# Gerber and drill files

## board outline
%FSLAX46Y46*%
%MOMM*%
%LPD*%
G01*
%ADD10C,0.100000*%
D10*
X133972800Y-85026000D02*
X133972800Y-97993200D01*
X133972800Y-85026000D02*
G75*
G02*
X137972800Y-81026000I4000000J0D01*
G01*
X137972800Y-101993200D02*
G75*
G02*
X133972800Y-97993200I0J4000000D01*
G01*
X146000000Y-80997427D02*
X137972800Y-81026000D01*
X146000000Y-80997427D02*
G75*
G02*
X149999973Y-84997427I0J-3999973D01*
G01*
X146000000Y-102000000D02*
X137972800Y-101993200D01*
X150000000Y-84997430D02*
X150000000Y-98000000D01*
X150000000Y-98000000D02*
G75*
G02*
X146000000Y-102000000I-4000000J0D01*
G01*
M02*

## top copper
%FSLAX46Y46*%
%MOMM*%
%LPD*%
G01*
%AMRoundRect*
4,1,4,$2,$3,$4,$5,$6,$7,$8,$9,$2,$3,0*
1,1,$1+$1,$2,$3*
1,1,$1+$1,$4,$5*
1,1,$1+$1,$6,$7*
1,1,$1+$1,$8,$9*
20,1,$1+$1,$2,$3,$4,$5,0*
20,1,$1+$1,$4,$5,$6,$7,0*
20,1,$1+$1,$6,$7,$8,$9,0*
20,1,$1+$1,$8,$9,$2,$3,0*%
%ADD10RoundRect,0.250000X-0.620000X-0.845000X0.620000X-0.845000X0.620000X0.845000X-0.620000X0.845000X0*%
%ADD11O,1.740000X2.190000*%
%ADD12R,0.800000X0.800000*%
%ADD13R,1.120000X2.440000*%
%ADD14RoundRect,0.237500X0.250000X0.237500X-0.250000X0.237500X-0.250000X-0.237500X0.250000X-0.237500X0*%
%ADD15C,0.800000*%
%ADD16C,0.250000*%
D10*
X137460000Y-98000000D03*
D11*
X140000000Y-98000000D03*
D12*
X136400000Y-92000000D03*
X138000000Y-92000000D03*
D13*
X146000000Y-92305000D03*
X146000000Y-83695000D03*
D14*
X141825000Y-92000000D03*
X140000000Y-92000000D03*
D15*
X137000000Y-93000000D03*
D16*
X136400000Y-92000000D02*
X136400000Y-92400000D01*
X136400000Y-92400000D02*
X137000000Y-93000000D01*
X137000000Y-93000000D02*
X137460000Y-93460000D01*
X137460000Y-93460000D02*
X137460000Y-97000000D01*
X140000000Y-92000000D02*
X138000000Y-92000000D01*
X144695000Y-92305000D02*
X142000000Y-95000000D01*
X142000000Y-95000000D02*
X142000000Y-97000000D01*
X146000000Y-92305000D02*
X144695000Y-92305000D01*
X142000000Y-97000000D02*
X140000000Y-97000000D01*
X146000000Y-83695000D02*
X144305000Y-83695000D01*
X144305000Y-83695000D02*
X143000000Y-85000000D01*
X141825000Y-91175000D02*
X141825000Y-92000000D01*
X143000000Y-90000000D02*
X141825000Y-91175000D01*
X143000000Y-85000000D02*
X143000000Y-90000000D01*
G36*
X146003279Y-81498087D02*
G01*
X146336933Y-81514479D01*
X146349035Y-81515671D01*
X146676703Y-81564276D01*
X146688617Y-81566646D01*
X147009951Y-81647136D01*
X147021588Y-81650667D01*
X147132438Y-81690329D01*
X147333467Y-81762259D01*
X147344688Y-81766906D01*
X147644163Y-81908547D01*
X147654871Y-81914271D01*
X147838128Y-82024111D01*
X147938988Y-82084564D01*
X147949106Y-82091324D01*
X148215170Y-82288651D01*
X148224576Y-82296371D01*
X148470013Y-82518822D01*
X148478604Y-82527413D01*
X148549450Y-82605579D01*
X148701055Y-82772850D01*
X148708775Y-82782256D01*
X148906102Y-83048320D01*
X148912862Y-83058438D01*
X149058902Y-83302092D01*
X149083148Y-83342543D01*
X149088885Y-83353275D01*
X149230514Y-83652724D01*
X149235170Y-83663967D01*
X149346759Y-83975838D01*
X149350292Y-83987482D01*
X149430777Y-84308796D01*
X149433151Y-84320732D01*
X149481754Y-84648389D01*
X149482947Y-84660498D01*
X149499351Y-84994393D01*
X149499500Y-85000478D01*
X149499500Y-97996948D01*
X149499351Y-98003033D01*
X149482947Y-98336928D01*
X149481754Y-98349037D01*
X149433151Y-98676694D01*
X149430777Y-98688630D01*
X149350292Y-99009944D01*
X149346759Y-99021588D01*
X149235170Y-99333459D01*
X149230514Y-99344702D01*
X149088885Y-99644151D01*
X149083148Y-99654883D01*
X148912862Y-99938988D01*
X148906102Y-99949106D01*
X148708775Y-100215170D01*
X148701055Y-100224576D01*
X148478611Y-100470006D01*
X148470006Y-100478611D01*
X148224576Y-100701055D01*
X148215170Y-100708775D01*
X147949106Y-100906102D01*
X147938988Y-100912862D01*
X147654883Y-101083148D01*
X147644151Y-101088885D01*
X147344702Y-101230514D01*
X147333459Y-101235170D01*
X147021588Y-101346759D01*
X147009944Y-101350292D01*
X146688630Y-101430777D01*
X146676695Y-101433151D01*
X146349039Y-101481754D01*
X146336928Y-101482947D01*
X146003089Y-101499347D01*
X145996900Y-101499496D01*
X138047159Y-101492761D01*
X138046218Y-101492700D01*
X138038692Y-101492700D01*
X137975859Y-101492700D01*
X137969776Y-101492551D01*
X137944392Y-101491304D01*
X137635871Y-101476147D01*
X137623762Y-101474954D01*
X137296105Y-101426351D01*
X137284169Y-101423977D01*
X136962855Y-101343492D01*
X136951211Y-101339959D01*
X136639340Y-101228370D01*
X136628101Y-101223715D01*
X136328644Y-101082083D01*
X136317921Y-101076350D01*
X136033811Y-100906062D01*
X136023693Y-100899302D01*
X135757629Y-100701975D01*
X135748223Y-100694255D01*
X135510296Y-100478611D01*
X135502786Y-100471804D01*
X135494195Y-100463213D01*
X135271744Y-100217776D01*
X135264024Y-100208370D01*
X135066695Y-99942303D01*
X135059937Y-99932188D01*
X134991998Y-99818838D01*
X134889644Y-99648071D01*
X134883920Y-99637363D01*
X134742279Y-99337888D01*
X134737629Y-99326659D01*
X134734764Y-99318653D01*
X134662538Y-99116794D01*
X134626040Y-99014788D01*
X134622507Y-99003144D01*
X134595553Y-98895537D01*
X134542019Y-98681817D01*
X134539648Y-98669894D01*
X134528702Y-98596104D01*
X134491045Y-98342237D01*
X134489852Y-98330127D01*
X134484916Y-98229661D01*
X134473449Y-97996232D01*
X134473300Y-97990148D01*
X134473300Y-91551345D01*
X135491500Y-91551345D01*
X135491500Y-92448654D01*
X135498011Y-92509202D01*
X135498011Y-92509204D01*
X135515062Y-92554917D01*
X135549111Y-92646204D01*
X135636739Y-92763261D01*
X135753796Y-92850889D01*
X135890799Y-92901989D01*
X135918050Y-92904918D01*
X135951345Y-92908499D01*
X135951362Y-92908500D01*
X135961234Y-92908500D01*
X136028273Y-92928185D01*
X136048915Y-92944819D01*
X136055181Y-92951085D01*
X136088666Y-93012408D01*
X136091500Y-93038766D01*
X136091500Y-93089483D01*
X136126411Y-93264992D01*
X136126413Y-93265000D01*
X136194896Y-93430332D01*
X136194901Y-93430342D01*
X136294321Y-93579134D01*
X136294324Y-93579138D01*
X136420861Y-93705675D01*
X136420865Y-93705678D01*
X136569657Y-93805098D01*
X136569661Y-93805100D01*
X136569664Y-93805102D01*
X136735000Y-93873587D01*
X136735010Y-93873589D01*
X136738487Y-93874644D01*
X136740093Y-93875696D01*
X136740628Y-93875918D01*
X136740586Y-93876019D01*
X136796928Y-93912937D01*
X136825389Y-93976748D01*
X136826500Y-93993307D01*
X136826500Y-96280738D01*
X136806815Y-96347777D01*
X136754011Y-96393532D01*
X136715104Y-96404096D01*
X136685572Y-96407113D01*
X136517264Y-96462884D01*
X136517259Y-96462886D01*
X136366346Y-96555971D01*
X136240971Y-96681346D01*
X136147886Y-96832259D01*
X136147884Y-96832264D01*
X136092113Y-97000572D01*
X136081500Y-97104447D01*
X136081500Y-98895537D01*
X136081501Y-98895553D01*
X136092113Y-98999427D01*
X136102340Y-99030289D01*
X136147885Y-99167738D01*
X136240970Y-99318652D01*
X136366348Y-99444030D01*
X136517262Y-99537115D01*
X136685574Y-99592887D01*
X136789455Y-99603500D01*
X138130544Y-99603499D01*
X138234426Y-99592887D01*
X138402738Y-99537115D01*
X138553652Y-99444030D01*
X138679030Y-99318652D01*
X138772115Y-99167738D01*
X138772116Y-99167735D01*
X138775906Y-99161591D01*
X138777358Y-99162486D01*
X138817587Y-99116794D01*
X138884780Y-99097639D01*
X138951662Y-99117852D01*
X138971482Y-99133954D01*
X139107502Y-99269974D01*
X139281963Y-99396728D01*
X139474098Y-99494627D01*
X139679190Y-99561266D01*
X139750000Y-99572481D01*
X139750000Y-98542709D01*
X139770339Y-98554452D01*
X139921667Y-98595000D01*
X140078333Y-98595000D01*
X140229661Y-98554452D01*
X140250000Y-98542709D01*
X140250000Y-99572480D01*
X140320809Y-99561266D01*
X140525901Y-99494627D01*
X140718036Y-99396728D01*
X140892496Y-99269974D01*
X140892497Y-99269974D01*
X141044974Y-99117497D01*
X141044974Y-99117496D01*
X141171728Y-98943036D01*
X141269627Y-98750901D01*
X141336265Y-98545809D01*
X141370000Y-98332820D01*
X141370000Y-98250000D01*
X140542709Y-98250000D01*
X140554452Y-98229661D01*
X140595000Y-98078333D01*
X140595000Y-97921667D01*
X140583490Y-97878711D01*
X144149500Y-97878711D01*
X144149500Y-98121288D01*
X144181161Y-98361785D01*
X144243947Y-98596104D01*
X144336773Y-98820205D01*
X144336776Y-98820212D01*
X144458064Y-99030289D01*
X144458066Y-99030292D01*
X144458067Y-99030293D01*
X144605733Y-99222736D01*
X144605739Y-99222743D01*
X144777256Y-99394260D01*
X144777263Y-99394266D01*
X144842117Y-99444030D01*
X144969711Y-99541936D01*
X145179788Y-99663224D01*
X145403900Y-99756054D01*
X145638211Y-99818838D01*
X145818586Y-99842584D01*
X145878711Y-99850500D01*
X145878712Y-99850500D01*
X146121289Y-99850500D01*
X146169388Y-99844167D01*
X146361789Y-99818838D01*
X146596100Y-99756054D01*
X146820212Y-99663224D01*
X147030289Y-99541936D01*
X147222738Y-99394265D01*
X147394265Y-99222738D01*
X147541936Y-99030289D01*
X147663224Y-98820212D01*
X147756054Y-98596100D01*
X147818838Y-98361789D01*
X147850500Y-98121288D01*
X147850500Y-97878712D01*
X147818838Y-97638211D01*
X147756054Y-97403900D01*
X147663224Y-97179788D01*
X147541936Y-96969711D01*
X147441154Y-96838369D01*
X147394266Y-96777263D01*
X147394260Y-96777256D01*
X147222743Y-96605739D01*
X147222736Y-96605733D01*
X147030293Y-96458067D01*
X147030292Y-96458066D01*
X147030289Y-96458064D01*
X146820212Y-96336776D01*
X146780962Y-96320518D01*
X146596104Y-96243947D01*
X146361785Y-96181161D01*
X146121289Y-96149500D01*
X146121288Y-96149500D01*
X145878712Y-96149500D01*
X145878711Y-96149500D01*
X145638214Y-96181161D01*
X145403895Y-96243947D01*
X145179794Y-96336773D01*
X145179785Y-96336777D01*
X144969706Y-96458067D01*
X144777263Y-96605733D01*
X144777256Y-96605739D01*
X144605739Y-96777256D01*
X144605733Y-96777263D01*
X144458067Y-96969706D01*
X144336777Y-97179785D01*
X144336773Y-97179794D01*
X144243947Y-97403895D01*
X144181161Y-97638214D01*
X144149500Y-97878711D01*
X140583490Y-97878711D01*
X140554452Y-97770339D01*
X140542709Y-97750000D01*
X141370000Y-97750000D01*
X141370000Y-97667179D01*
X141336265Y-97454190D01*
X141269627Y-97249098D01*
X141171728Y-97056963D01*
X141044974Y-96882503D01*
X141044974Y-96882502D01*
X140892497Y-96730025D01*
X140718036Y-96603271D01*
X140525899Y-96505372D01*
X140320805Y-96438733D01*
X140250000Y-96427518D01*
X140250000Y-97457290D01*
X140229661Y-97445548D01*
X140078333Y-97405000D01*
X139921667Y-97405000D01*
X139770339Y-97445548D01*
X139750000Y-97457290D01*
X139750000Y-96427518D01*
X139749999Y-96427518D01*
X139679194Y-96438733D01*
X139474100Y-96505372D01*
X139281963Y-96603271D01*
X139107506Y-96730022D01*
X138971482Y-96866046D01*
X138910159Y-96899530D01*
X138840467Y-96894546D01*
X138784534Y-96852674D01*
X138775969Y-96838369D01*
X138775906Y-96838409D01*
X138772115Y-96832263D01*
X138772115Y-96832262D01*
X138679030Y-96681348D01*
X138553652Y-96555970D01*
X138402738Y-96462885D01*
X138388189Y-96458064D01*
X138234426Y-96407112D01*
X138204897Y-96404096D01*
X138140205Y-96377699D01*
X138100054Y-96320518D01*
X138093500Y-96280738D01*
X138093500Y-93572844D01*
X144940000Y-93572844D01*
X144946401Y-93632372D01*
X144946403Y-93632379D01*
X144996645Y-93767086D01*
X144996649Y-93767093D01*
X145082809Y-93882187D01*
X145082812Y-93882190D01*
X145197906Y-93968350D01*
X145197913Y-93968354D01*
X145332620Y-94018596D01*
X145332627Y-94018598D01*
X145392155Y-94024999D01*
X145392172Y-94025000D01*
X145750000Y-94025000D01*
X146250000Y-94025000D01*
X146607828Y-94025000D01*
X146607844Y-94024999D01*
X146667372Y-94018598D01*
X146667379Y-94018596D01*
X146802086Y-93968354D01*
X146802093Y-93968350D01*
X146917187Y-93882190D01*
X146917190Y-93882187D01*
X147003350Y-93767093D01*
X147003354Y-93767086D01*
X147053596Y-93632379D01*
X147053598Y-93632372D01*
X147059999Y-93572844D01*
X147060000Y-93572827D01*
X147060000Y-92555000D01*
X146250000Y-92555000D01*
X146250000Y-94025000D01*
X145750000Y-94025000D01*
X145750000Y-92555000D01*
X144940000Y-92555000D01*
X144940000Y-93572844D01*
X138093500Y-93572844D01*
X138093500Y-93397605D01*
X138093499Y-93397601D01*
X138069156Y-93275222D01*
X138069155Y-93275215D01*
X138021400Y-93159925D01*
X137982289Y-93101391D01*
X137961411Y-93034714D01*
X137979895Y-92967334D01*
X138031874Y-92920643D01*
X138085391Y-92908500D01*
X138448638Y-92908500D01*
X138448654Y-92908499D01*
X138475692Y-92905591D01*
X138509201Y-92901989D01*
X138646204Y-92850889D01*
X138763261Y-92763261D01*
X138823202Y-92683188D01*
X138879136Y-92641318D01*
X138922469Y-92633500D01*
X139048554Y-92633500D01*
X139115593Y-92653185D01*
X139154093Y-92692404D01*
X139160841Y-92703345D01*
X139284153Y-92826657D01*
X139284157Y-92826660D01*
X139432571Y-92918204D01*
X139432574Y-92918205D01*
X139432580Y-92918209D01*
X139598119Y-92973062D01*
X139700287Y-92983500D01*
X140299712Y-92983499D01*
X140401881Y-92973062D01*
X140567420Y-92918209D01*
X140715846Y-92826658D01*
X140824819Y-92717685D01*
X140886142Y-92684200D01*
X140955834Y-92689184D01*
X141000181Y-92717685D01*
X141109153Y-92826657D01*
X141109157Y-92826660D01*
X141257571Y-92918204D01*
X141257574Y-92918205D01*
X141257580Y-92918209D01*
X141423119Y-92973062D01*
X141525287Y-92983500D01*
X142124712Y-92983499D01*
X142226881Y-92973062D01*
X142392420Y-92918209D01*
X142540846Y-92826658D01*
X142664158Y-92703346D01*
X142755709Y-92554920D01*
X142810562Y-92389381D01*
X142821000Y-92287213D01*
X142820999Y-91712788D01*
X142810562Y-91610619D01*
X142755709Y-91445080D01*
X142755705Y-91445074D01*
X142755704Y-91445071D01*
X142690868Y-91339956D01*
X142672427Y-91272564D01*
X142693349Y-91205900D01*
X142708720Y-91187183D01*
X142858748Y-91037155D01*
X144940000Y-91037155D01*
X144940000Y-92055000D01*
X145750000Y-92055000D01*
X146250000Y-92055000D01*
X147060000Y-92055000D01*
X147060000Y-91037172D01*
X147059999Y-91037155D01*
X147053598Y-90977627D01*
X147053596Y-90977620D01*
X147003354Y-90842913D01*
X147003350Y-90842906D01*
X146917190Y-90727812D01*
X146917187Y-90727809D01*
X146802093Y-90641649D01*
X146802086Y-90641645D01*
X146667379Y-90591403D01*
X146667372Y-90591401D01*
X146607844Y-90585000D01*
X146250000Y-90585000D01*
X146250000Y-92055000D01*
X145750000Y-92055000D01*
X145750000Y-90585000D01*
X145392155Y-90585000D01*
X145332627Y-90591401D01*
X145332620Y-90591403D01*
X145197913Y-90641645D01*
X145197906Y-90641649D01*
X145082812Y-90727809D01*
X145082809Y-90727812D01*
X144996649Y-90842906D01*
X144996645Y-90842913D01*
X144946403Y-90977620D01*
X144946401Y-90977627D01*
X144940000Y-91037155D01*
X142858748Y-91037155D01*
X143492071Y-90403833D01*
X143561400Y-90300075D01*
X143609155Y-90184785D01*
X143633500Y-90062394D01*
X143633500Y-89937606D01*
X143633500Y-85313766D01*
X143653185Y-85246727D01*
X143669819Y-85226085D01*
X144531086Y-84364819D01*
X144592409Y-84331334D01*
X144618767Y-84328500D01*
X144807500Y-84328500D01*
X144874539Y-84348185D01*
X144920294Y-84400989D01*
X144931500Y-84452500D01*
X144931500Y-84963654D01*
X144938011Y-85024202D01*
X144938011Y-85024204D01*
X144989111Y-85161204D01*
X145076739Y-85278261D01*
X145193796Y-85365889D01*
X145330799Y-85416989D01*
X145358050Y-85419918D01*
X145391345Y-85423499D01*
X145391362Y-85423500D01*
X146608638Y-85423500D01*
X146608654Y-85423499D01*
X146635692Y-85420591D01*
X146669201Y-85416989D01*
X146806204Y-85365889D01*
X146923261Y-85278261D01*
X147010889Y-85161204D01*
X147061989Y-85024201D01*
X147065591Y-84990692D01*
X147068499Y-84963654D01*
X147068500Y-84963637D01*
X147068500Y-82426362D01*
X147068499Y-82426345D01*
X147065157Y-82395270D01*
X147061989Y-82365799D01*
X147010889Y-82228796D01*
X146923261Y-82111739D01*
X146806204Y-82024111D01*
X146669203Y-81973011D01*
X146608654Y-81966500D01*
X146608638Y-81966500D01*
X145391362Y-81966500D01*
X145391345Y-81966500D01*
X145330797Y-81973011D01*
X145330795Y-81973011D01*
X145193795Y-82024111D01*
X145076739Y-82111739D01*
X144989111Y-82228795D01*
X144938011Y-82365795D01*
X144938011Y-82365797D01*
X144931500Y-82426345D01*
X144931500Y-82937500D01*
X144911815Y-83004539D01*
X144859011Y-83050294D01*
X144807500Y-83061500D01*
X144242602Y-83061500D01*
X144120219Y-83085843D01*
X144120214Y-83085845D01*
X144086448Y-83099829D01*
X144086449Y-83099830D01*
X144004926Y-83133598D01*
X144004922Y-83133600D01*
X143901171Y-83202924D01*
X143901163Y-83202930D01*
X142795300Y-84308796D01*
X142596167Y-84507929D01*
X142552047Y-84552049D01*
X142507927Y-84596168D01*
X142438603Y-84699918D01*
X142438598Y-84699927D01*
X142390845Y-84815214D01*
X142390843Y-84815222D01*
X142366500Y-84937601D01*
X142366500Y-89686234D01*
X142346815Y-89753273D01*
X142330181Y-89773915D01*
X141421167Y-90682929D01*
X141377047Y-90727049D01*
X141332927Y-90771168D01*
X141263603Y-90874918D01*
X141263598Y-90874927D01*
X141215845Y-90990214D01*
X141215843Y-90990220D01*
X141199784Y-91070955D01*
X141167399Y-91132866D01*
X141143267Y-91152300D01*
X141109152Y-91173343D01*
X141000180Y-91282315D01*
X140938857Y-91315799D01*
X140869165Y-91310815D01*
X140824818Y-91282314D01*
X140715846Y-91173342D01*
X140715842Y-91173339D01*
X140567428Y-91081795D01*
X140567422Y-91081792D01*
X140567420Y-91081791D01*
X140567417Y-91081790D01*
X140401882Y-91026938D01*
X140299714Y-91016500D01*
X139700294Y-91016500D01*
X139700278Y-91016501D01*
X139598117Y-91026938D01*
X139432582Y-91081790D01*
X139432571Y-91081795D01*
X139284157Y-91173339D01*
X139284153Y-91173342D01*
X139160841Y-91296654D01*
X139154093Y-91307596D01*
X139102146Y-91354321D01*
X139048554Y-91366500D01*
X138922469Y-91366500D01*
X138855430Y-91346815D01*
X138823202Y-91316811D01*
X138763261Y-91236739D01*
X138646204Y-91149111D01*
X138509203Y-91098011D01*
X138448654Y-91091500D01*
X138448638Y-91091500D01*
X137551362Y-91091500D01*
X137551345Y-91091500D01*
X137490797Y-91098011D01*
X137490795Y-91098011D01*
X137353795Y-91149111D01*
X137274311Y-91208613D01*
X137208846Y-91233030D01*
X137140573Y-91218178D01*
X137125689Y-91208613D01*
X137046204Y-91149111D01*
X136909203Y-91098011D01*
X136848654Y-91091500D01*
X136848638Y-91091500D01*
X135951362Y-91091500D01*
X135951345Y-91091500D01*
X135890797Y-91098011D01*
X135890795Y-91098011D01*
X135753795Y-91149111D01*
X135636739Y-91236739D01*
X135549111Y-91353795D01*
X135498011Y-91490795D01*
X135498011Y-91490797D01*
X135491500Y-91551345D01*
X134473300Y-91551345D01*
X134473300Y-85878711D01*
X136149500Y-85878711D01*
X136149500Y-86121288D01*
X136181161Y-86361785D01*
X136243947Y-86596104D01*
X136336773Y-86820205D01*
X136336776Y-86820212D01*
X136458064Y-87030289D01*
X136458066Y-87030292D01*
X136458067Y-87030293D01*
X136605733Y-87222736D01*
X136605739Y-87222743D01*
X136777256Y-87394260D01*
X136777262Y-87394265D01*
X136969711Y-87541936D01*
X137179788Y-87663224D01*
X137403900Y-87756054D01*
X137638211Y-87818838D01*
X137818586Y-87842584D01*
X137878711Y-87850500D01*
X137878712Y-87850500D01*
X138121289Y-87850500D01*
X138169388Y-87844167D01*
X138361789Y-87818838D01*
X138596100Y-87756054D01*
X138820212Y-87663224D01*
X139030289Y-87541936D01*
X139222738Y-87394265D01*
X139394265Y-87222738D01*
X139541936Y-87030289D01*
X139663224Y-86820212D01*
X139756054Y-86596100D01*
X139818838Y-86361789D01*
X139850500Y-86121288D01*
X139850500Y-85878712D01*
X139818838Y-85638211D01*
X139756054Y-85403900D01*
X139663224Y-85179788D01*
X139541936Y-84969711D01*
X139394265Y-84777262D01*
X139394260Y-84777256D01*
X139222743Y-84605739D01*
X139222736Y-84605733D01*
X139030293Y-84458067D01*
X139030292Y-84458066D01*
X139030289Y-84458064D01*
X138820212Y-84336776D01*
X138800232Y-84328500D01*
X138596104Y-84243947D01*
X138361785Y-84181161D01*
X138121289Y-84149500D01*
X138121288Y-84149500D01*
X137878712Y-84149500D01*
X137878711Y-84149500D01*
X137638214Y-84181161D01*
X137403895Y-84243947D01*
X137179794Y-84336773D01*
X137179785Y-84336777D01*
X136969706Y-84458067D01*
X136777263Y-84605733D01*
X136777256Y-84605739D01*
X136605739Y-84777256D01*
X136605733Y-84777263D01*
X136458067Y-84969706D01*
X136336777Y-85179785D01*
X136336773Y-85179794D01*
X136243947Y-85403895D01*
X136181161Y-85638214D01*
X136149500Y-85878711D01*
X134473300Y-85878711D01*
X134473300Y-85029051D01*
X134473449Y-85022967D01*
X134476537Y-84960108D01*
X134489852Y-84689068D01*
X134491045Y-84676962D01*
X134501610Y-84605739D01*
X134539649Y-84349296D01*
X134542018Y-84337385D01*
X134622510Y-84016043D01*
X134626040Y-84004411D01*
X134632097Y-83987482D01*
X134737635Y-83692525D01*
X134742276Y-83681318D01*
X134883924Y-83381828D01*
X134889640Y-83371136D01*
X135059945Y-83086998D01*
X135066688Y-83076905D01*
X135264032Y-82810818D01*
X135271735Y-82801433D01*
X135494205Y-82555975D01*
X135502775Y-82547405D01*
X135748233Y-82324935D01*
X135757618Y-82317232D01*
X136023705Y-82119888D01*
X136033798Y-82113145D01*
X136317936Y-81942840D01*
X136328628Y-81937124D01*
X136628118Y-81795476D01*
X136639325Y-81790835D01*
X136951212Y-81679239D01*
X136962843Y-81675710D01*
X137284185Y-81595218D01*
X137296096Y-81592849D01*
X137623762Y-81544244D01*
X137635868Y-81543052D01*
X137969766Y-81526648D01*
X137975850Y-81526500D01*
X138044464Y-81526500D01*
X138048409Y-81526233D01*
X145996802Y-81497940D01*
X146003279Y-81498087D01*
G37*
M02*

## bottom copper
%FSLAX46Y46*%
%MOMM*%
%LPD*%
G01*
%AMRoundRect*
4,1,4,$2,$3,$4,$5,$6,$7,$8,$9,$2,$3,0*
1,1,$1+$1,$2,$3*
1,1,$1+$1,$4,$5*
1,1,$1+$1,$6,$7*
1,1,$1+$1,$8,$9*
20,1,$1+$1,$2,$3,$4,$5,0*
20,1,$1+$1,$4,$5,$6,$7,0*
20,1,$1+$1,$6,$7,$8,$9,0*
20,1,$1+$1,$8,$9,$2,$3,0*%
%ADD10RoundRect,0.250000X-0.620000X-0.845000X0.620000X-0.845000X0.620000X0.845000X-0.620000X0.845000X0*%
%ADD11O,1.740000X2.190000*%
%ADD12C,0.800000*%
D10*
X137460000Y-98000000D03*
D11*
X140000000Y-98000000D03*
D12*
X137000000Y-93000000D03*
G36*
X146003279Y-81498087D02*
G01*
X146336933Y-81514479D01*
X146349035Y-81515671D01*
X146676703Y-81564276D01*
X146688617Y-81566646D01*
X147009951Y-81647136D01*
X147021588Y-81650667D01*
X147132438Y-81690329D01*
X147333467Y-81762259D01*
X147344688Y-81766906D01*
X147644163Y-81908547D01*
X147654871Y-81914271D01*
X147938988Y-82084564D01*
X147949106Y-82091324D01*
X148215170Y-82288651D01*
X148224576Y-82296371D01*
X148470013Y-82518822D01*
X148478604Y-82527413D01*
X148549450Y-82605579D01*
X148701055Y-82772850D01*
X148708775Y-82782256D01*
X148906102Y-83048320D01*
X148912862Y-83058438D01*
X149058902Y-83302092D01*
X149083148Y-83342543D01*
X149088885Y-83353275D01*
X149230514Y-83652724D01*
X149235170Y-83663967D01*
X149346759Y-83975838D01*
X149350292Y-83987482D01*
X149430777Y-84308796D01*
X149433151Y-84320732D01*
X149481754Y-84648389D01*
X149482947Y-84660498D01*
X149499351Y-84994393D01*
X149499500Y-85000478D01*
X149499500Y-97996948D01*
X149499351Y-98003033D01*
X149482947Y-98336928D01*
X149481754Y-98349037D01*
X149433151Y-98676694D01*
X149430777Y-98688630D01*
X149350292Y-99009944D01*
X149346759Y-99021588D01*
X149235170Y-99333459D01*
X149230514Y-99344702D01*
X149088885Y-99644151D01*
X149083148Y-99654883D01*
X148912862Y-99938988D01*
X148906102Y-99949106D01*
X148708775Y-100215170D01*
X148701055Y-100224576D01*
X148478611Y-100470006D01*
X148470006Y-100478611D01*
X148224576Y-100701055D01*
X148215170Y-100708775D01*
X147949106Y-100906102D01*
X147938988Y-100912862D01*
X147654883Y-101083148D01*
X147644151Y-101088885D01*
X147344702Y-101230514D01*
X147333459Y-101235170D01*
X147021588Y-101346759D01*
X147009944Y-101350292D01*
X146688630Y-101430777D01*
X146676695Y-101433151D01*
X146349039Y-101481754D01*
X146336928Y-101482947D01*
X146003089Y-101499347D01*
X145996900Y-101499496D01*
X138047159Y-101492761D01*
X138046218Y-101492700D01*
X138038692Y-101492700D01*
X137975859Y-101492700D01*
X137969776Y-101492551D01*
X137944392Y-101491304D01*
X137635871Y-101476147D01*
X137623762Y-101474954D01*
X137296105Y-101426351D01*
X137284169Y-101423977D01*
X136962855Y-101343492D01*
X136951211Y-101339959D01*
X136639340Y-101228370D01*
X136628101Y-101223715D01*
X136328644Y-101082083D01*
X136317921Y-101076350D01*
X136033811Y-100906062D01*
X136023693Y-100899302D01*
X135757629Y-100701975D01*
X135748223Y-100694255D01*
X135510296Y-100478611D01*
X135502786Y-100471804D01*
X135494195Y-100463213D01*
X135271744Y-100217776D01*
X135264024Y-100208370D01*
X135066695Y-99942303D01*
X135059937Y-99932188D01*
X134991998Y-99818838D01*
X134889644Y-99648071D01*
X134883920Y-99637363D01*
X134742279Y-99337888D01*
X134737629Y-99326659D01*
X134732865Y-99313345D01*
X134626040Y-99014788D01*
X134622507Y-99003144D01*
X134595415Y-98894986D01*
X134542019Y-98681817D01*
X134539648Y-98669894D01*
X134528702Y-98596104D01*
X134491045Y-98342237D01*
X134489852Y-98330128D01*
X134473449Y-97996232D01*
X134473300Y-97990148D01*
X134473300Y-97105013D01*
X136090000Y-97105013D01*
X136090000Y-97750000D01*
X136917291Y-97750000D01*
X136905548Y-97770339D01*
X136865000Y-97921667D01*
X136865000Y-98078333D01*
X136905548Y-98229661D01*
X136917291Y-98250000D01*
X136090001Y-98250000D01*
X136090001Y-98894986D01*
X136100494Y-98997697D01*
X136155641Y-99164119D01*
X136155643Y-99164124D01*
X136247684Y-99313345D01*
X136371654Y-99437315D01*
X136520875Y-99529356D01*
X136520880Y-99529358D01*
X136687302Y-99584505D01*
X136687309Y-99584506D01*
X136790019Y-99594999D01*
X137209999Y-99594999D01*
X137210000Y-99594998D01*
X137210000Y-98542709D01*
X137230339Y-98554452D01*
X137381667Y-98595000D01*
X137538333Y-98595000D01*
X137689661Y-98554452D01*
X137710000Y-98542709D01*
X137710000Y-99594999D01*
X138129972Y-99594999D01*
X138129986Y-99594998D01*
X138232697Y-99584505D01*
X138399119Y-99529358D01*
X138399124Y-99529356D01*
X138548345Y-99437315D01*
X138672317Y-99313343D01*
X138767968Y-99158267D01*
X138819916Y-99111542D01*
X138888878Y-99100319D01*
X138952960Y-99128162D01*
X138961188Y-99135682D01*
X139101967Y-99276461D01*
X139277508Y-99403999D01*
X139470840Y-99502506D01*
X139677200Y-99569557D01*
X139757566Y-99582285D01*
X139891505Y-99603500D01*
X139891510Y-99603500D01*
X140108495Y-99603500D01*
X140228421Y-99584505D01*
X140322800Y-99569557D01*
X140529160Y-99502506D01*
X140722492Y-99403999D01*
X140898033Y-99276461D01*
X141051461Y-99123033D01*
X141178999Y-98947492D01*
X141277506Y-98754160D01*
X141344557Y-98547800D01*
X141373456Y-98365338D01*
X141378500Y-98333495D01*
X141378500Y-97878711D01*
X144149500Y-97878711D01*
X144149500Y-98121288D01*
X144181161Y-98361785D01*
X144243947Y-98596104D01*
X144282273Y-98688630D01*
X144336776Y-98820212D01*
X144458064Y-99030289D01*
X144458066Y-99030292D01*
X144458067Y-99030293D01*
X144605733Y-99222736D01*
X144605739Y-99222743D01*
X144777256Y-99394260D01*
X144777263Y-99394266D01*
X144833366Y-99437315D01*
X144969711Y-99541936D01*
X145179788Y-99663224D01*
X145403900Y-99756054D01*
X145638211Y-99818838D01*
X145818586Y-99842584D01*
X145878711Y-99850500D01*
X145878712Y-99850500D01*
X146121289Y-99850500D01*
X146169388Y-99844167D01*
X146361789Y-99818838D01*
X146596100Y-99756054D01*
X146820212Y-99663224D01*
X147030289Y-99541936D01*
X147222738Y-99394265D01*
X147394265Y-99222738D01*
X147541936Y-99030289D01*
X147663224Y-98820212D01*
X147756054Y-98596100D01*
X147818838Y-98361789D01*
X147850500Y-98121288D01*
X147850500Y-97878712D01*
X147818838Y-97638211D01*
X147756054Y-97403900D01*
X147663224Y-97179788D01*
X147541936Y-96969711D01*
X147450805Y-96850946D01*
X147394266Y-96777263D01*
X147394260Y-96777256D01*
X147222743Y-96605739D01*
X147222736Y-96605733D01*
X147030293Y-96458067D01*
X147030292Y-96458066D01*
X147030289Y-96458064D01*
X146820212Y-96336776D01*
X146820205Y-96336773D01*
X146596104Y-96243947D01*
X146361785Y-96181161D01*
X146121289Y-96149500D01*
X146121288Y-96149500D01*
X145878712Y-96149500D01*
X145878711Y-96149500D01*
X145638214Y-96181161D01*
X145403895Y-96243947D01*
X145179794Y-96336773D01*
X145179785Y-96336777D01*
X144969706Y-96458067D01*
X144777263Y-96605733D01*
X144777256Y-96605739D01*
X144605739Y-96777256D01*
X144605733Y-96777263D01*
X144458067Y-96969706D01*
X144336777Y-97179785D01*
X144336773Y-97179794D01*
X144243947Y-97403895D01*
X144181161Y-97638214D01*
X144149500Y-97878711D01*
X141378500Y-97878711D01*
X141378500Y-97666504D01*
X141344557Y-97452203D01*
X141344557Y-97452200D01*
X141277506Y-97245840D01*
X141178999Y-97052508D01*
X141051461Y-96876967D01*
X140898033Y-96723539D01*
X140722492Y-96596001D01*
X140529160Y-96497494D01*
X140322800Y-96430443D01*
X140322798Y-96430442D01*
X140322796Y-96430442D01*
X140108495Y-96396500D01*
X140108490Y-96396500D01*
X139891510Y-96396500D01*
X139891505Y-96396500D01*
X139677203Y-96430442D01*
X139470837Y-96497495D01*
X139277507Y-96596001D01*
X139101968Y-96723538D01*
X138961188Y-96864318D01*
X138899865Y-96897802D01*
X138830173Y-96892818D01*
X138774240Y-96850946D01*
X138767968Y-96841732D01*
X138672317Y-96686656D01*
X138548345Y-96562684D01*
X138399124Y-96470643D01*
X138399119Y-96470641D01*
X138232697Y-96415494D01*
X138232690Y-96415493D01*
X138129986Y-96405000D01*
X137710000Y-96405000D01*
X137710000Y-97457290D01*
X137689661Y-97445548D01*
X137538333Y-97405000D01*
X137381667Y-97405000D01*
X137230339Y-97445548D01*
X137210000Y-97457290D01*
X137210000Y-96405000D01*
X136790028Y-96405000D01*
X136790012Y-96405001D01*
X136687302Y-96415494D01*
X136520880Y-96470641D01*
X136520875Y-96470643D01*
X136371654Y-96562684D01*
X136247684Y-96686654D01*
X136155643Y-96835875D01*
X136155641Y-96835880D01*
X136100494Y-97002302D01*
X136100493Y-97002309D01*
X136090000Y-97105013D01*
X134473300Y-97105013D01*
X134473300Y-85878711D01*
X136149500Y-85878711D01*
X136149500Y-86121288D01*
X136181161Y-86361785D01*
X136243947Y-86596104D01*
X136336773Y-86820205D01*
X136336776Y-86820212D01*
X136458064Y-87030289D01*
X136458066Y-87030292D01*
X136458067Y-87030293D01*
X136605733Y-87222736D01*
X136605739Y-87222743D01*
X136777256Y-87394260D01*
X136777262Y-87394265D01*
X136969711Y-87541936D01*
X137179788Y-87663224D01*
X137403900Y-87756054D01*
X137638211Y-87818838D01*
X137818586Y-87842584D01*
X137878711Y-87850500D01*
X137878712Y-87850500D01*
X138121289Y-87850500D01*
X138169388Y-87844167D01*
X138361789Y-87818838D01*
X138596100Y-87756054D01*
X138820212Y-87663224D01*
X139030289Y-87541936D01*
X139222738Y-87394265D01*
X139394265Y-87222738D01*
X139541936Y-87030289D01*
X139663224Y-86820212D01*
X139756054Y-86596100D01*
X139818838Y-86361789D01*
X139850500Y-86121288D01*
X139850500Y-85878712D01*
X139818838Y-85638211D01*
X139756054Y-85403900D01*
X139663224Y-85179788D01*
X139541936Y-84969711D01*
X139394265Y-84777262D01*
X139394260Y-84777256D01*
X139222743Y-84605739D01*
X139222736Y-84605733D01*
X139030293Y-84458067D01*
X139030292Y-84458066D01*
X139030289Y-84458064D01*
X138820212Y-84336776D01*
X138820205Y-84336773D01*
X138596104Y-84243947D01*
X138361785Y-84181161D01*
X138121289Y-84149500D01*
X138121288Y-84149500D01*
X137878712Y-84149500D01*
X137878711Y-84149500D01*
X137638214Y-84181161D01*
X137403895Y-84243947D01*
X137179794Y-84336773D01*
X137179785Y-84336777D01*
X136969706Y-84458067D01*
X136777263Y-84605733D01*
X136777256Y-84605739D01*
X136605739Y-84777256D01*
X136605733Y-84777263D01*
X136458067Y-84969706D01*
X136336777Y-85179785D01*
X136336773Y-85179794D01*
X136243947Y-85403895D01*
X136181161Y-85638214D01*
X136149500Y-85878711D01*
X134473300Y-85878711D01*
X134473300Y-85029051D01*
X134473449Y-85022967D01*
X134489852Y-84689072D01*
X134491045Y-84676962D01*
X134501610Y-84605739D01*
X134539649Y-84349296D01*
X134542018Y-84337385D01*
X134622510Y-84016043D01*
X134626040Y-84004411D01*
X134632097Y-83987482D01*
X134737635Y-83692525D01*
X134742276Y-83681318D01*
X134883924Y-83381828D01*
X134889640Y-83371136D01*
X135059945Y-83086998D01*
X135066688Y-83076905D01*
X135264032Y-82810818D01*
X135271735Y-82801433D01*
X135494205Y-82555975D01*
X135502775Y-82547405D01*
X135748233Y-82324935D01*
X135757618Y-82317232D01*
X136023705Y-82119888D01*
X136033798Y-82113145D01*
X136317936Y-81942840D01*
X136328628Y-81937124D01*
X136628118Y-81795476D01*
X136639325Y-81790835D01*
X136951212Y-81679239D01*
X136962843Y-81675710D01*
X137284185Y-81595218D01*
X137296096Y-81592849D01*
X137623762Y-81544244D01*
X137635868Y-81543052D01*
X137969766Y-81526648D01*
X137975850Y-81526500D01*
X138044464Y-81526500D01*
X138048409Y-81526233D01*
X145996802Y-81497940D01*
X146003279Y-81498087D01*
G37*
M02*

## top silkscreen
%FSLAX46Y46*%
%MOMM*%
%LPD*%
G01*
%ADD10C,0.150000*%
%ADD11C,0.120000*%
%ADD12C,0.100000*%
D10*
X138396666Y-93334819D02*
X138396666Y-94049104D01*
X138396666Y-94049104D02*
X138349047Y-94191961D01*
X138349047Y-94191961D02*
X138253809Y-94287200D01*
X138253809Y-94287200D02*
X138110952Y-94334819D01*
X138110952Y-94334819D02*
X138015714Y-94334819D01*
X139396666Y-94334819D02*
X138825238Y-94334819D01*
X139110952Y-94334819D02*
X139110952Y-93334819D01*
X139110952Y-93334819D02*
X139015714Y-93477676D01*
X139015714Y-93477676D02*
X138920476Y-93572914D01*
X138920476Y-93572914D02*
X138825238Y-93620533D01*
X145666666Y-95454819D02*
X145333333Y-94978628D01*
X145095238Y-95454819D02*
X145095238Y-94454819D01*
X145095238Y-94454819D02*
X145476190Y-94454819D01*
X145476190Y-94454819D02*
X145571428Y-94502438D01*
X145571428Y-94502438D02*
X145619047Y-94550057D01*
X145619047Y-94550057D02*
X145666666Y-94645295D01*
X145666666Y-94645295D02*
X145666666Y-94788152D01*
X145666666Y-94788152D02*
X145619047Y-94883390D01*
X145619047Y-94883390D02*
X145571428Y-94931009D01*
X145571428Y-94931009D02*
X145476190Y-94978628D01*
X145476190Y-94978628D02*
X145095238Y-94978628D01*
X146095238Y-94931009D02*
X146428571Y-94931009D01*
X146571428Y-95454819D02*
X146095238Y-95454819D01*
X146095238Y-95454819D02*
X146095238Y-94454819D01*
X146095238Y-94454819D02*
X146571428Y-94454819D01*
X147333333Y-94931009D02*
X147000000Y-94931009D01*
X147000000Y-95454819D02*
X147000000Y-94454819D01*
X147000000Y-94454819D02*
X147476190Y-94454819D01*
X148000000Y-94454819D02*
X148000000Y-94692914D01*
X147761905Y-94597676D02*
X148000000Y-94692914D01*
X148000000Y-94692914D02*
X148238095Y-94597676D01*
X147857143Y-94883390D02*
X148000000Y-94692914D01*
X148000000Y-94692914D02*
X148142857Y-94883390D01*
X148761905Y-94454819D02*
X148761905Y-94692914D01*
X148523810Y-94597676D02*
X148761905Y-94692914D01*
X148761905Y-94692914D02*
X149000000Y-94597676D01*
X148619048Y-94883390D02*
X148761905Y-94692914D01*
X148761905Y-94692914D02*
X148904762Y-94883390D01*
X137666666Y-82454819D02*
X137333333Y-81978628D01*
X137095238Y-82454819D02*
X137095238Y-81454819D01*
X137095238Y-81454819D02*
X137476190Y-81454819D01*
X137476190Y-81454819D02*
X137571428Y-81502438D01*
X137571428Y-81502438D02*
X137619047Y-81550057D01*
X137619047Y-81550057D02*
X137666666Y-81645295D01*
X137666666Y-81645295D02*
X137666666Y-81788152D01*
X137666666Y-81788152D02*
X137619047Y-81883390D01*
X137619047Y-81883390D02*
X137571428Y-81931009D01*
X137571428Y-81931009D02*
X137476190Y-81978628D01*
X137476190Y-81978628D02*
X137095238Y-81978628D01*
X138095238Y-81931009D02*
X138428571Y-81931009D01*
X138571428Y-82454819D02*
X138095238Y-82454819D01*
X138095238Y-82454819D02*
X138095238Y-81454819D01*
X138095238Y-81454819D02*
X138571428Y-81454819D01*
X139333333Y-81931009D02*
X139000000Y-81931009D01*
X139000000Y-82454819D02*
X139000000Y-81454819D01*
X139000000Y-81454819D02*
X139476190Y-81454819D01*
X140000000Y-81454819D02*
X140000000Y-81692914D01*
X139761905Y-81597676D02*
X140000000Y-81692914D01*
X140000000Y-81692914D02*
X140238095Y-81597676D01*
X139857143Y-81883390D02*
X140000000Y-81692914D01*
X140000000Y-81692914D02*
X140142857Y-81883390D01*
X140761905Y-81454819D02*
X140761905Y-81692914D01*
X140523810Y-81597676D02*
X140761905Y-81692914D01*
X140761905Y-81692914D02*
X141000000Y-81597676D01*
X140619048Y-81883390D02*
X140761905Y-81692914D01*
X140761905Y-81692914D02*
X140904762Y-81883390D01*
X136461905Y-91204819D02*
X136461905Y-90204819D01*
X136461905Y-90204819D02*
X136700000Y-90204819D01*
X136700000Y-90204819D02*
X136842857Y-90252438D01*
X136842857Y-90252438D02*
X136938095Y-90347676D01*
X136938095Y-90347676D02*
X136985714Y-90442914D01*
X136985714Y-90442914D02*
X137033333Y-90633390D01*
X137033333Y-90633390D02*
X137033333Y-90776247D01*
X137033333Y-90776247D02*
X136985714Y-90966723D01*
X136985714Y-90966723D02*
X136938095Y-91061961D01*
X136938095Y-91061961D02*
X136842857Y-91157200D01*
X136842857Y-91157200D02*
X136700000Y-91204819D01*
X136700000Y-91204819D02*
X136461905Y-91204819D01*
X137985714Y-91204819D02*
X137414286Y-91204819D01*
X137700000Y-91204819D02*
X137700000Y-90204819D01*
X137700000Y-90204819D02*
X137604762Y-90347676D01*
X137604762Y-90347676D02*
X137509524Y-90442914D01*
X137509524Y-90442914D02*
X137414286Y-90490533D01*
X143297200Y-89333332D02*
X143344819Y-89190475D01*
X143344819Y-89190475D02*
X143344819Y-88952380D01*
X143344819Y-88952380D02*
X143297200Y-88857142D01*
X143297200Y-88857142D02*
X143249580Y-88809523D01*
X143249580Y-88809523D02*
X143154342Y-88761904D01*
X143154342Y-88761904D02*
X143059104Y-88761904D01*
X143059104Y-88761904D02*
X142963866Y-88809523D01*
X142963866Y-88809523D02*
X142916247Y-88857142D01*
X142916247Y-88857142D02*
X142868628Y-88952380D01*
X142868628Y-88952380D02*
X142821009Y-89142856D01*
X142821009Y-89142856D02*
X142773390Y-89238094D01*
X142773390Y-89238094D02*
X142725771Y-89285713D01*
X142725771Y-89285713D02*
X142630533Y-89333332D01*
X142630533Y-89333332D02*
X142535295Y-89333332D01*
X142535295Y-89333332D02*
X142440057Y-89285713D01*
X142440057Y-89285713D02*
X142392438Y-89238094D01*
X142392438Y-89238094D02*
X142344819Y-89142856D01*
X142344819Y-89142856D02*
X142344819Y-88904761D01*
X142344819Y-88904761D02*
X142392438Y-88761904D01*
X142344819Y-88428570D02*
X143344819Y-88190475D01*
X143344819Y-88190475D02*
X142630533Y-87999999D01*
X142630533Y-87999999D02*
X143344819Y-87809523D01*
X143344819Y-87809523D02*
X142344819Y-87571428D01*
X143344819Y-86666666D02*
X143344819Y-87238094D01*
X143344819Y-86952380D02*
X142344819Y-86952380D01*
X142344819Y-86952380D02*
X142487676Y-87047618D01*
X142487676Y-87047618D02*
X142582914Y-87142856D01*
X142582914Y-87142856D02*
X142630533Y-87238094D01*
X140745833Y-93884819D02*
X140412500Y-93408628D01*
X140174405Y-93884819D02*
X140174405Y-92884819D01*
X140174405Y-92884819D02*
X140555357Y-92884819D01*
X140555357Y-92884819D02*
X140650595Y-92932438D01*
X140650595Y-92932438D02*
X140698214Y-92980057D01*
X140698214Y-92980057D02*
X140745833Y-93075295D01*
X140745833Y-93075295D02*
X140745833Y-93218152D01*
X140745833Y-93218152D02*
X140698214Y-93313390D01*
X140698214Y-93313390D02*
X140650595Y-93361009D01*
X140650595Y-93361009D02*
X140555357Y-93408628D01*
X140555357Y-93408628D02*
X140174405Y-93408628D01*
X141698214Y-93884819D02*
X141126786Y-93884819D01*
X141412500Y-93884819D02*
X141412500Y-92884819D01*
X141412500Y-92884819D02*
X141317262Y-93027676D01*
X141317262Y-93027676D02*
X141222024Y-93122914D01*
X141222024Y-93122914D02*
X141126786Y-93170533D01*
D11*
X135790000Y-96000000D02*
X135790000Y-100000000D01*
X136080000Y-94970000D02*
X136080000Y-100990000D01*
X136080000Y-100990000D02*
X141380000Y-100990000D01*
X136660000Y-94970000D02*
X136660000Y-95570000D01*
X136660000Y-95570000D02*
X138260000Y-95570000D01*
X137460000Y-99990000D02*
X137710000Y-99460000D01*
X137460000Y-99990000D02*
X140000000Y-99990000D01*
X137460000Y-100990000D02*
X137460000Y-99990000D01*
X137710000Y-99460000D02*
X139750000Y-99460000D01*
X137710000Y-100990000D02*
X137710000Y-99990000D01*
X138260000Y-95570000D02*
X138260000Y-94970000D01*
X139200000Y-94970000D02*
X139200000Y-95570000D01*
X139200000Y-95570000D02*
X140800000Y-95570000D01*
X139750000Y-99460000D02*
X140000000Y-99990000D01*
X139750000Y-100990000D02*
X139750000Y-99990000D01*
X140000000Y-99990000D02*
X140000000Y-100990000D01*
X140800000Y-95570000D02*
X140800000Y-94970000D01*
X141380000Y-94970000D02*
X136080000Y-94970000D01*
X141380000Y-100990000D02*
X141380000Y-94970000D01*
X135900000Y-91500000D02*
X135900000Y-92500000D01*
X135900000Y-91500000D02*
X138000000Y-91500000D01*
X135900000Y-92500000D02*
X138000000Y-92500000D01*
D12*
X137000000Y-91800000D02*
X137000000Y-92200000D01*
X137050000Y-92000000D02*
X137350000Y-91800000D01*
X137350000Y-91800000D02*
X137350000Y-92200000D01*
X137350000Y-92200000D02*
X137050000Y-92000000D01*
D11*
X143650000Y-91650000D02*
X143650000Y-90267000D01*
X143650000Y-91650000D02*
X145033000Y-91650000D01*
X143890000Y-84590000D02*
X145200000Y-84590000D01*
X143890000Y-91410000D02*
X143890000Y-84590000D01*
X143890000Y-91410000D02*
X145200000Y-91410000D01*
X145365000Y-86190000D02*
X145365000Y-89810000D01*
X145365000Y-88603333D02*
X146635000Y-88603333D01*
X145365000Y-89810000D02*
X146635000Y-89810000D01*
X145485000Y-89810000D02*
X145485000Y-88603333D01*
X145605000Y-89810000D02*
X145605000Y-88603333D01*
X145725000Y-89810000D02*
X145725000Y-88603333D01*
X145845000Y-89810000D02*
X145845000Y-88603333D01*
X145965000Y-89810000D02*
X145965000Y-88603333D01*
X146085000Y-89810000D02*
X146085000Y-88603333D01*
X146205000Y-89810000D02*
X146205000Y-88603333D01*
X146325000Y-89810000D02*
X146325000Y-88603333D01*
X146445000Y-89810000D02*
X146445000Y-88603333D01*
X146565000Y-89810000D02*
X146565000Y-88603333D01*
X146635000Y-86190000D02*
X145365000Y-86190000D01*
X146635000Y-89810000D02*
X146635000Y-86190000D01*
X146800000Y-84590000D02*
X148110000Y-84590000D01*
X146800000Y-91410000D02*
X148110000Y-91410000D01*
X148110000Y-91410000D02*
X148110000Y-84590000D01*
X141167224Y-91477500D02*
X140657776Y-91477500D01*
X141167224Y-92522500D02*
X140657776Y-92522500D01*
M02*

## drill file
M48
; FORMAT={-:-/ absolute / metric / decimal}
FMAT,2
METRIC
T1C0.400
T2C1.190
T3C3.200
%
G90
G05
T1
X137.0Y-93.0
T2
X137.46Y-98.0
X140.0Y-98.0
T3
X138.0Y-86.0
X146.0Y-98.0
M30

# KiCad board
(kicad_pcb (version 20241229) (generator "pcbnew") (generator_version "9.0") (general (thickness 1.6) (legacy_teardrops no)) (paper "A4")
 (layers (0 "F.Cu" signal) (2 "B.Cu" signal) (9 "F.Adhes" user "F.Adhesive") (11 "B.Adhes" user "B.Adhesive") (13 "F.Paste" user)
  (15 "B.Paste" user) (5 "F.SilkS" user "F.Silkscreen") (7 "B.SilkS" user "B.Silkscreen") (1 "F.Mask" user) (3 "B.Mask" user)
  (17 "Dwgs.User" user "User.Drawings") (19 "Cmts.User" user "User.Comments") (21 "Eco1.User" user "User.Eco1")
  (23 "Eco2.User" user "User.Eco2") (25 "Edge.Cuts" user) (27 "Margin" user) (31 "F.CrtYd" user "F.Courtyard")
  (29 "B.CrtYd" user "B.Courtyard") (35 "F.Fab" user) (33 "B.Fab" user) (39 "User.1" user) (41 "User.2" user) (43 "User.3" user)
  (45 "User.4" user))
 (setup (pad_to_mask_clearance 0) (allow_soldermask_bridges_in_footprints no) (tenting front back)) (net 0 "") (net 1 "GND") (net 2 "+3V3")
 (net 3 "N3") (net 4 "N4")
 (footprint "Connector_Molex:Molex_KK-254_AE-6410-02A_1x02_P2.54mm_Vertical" (layer "F.Cu") (at 137.46 98)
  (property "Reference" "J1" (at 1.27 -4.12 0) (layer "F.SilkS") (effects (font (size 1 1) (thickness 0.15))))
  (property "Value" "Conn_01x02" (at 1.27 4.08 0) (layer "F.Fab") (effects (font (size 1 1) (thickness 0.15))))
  (fp_line (start -1.67 -2) (end -1.67 2) (stroke (width 0.12) (type solid)) (layer "F.SilkS"))
  (fp_line (start -1.38 -3.03) (end -1.38 2.99) (stroke (width 0.12) (type solid)) (layer "F.SilkS"))
  (fp_line (start -1.38 2.99) (end 3.92 2.99) (stroke (width 0.12) (type solid)) (layer "F.SilkS"))
  (fp_line (start -0.8 -3.03) (end -0.8 -2.43) (stroke (width 0.12) (type solid)) (layer "F.SilkS"))
  (fp_line (start -0.8 -2.43) (end 0.8 -2.43) (stroke (width 0.12) (type solid)) (layer "F.SilkS"))
  (fp_line (start 0 1.99) (end 0.25 1.46) (stroke (width 0.12) (type solid)) (layer "F.SilkS"))
  (fp_line (start 0 1.99) (end 2.54 1.99) (stroke (width 0.12) (type solid)) (layer "F.SilkS"))
  (fp_line (start 0 2.99) (end 0 1.99) (stroke (width 0.12) (type solid)) (layer "F.SilkS"))
  (fp_line (start 0.25 1.46) (end 2.29 1.46) (stroke (width 0.12) (type solid)) (layer "F.SilkS"))
  (fp_line (start 0.25 2.99) (end 0.25 1.99) (stroke (width 0.12) (type solid)) (layer "F.SilkS"))
  (fp_line (start 0.8 -2.43) (end 0.8 -3.03) (stroke (width 0.12) (type solid)) (layer "F.SilkS"))
  (fp_line (start 1.74 -3.03) (end 1.74 -2.43) (stroke (width 0.12) (type solid)) (layer "F.SilkS"))
  (fp_line (start 1.74 -2.43) (end 3.34 -2.43) (stroke (width 0.12) (type solid)) (layer "F.SilkS"))
  (fp_line (start 2.29 1.46) (end 2.54 1.99) (stroke (width 0.12) (type solid)) (layer "F.SilkS"))
  (fp_line (start 2.29 2.99) (end 2.29 1.99) (stroke (width 0.12) (type solid)) (layer "F.SilkS"))
  (fp_line (start 2.54 1.99) (end 2.54 2.99) (stroke (width 0.12) (type solid)) (layer "F.SilkS"))
  (fp_line (start 3.34 -2.43) (end 3.34 -3.03) (stroke (width 0.12) (type solid)) (layer "F.SilkS"))
  (fp_line (start 3.92 -3.03) (end -1.38 -3.03) (stroke (width 0.12) (type solid)) (layer "F.SilkS"))
  (fp_line (start 3.92 2.99) (end 3.92 -3.03) (stroke (width 0.12) (type solid)) (layer "F.SilkS"))
  (pad "1" thru_hole roundrect (at 0 0) (size 1.74 2.19) (drill 1.19) (layers "*.Cu" "*.Mask") (remove_unused_layers no)
   (roundrect_rratio 0.143678) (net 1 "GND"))
  (pad "2" thru_hole oval (at 2.54 0) (size 1.74 2.19) (drill 1.19) (layers "*.Cu" "*.Mask") (remove_unused_layers no) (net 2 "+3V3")))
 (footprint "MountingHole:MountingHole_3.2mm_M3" (layer "F.Cu") (at 146 98)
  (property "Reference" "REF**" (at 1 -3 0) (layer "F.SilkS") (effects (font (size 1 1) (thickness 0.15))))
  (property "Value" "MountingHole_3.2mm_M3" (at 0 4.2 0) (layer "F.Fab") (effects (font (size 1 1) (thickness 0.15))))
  (pad "" np_thru_hole circle (at 0 0) (size 3.2 3.2) (drill 3.2) (layers "*.Cu" "*.Mask")))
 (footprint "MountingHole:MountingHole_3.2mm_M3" (layer "F.Cu") (at 138 86)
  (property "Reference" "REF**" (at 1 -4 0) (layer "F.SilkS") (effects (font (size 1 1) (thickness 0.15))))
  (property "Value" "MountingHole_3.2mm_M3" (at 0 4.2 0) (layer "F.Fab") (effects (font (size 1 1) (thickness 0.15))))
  (pad "" np_thru_hole circle (at 0 0) (size 3.2 3.2) (drill 3.2) (layers "*.Cu" "*.Mask")))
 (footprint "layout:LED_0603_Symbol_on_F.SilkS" (layer "F.Cu") (at 137.2 92)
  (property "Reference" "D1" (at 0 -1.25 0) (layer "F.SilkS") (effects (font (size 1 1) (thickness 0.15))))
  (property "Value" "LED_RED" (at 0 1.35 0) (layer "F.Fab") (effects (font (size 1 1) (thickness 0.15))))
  (fp_line (start -1.3 -0.5) (end -1.3 0.5) (stroke (width 0.12) (type solid)) (layer "F.SilkS"))
  (fp_line (start -1.3 -0.5) (end 0.8 -0.5) (stroke (width 0.12) (type solid)) (layer "F.SilkS"))
  (fp_line (start -1.3 0.5) (end 0.8 0.5) (stroke (width 0.12) (type solid)) (layer "F.SilkS"))
  (fp_line (start -0.2 -0.2) (end -0.2 0.2) (stroke (width 0.1) (type solid)) (layer "F.SilkS"))
  (fp_line (start -0.15 0) (end 0.15 -0.2) (stroke (width 0.1) (type solid)) (layer "F.SilkS"))
  (fp_line (start 0.15 -0.2) (end 0.15 0.2) (stroke (width 0.1) (type solid)) (layer "F.SilkS"))
  (fp_line (start 0.15 0.2) (end -0.15 0) (stroke (width 0.1) (type solid)) (layer "F.SilkS"))
  (pad "1" smd rect (at -0.8 0 180) (size 0.8 0.8) (layers "F.Cu" "F.Mask" "F.Paste") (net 1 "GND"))
  (pad "2" smd rect (at 0.8 0 180) (size 0.8 0.8) (layers "F.Cu" "F.Mask" "F.Paste") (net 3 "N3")))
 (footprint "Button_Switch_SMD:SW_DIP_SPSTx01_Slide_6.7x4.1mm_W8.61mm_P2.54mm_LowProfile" (layer "F.Cu") (at 146 88 90)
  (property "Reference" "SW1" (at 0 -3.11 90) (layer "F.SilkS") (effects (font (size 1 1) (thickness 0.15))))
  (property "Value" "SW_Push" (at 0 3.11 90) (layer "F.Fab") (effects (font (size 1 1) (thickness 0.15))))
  (fp_line (start -3.65 -2.35) (end -2.267 -2.35) (stroke (width 0.12) (type solid)) (layer "F.SilkS"))
  (fp_line (start -3.65 -2.35) (end -3.65 -0.967) (stroke (width 0.12) (type solid)) (layer "F.SilkS"))
  (fp_line (start 3.41 -2.11) (end 3.41 -0.8) (stroke (width 0.12) (type solid)) (layer "F.SilkS"))
  (fp_line (start -3.41 -2.11) (end 3.41 -2.11) (stroke (width 0.12) (type solid)) (layer "F.SilkS"))
  (fp_line (start -3.41 -2.11) (end -3.41 -0.8) (stroke (width 0.12) (type solid)) (layer "F.SilkS"))
  (fp_line (start 1.81 -0.635) (end -1.81 -0.635) (stroke (width 0.12) (type solid)) (layer "F.SilkS"))
  (fp_line (start -0.603333 -0.635) (end -0.603333 0.635) (stroke (width 0.12) (type solid)) (layer "F.SilkS"))
  (fp_line (start -1.81 -0.635) (end -1.81 0.635) (stroke (width 0.12) (type solid)) (layer "F.SilkS"))
  (fp_line (start -1.81 -0.515) (end -0.603333 -0.515) (stroke (width 0.12) (type solid)) (layer "F.SilkS"))
  (fp_line (start -1.81 -0.395) (end -0.603333 -0.395) (stroke (width 0.12) (type solid)) (layer "F.SilkS"))
  (fp_line (start -1.81 -0.275) (end -0.603333 -0.275) (stroke (width 0.12) (type solid)) (layer "F.SilkS"))
  (fp_line (start -1.81 -0.155) (end -0.603333 -0.155) (stroke (width 0.12) (type solid)) (layer "F.SilkS"))
  (fp_line (start -1.81 -0.035) (end -0.603333 -0.035) (stroke (width 0.12) (type solid)) (layer "F.SilkS"))
  (fp_line (start -1.81 0.085) (end -0.603333 0.085) (stroke (width 0.12) (type solid)) (layer "F.SilkS"))
  (fp_line (start -1.81 0.205) (end -0.603333 0.205) (stroke (width 0.12) (type solid)) (layer "F.SilkS"))
  (fp_line (start -1.81 0.325) (end -0.603333 0.325) (stroke (width 0.12) (type solid)) (layer "F.SilkS"))
  (fp_line (start -1.81 0.445) (end -0.603333 0.445) (stroke (width 0.12) (type solid)) (layer "F.SilkS"))
  (fp_line (start -1.81 0.565) (end -0.603333 0.565) (stroke (width 0.12) (type solid)) (layer "F.SilkS"))
  (fp_line (start 1.81 0.635) (end 1.81 -0.635) (stroke (width 0.12) (type solid)) (layer "F.SilkS"))
  (fp_line (start -1.81 0.635) (end 1.81 0.635) (stroke (width 0.12) (type solid)) (layer "F.SilkS"))
  (fp_line (start 3.41 0.8) (end 3.41 2.11) (stroke (width 0.12) (type solid)) (layer "F.SilkS"))
  (fp_line (start -3.41 0.8) (end -3.41 2.11) (stroke (width 0.12) (type solid)) (layer "F.SilkS"))
  (fp_line (start -3.41 2.11) (end 3.41 2.11) (stroke (width 0.12) (type solid)) (layer "F.SilkS"))
  (pad "1" smd rect (at -4.305 0 90) (size 2.44 1.12) (layers "F.Cu" "F.Mask" "F.Paste") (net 2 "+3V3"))
  (pad "2" smd rect (at 4.305 0 90) (size 2.44 1.12) (layers "F.Cu" "F.Mask" "F.Paste") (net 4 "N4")))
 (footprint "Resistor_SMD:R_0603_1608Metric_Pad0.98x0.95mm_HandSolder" (layer "F.Cu") (at 140.9125 92 180)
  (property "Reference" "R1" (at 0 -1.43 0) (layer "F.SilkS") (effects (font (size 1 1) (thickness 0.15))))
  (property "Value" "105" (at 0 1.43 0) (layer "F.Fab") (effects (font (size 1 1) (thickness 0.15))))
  (fp_line (start -0.254724 0.5225) (end 0.254724 0.5225) (stroke (width 0.12) (type solid)) (layer "F.SilkS"))
  (fp_line (start -0.254724 -0.5225) (end 0.254724 -0.5225) (stroke (width 0.12) (type solid)) (layer "F.SilkS"))
  (pad "1" smd roundrect (at -0.9125 0 180) (size 0.975 0.95) (layers "F.Cu" "F.Mask" "F.Paste") (roundrect_rratio 0.25) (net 4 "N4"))
  (pad "2" smd roundrect (at 0.9125 0 180) (size 0.975 0.95) (layers "F.Cu" "F.Mask" "F.Paste") (roundrect_rratio 0.25) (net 3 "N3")))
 (gr_line (start 133.9728 85.026) (end 133.9728 97.9932) (stroke (width 0.1) (type default)) (layer "Edge.Cuts"))
 (gr_arc (start 133.9728 85.026) (mid 135.144373 82.197573) (end 137.9728 81.026) (stroke (width 0.1) (type solid)) (layer "Edge.Cuts"))
 (gr_arc (start 137.9728 101.9932) (mid 135.144373 100.821627) (end 133.9728 97.9932) (stroke (width 0.1) (type solid)) (layer "Edge.Cuts"))
 (gr_line (start 146 80.997427) (end 137.9728 81.026) (stroke (width 0.1) (type default)) (layer "Edge.Cuts"))
 (gr_arc (start 146 80.997427) (mid 148.828427 82.169) (end 150 84.997427) (stroke (width 0.1) (type solid)) (layer "Edge.Cuts"))
 (gr_line (start 146 102) (end 137.9728 101.9932) (stroke (width 0.1) (type default)) (layer "Edge.Cuts"))
 (gr_line (start 150 84.99743) (end 150 98) (stroke (width 0.1) (type default)) (layer "Edge.Cuts"))
 (gr_arc (start 150 98) (mid 148.828427 100.828427) (end 146 102) (stroke (width 0.1) (type solid)) (layer "Edge.Cuts"))
 (segment (start 136.4 92) (end 136.4 92.4) (width 0.25) (layer "F.Cu") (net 1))
 (segment (start 136.4 92.4) (end 137 93) (width 0.25) (layer "F.Cu") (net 1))
 (segment (start 137 93) (end 137.46 93.46) (width 0.25) (layer "F.Cu") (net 1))
 (segment (start 137.46 93.46) (end 137.46 97) (width 0.25) (layer "F.Cu") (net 1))
 (via (at 137 93) (size 0.8) (drill 0.4) (layers "F.Cu" "B.Cu") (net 1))
 (segment (start 140 92) (end 138 92) (width 0.25) (layer "F.Cu") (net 3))
 (segment (start 144.695 92.305) (end 142 95) (width 0.25) (layer "F.Cu") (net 2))
 (segment (start 142 95) (end 142 97) (width 0.25) (layer "F.Cu") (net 2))
 (segment (start 146 92.305) (end 144.695 92.305) (width 0.25) (layer "F.Cu") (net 2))
 (segment (start 142 97) (end 140 97) (width 0.25) (layer "F.Cu") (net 2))
 (segment (start 146 83.695) (end 144.305 83.695) (width 0.25) (layer "F.Cu") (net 4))
 (segment (start 144.305 83.695) (end 143 85) (width 0.25) (layer "F.Cu") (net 4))
 (segment (start 141.825 91.175) (end 141.825 92) (width 0.25) (layer "F.Cu") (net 4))
 (segment (start 143 90) (end 141.825 91.175) (width 0.25) (layer "F.Cu") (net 4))
 (segment (start 143 85) (end 143 90) (width 0.25) (layer "F.Cu") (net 4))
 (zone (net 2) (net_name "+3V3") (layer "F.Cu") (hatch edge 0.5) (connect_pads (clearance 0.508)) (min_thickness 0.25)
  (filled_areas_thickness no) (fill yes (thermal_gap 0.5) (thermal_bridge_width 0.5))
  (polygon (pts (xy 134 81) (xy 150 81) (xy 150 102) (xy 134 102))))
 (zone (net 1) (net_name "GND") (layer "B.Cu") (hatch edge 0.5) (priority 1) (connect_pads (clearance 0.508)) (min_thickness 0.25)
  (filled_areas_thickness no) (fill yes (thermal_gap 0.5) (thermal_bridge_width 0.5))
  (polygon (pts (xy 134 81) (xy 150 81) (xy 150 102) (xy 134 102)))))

